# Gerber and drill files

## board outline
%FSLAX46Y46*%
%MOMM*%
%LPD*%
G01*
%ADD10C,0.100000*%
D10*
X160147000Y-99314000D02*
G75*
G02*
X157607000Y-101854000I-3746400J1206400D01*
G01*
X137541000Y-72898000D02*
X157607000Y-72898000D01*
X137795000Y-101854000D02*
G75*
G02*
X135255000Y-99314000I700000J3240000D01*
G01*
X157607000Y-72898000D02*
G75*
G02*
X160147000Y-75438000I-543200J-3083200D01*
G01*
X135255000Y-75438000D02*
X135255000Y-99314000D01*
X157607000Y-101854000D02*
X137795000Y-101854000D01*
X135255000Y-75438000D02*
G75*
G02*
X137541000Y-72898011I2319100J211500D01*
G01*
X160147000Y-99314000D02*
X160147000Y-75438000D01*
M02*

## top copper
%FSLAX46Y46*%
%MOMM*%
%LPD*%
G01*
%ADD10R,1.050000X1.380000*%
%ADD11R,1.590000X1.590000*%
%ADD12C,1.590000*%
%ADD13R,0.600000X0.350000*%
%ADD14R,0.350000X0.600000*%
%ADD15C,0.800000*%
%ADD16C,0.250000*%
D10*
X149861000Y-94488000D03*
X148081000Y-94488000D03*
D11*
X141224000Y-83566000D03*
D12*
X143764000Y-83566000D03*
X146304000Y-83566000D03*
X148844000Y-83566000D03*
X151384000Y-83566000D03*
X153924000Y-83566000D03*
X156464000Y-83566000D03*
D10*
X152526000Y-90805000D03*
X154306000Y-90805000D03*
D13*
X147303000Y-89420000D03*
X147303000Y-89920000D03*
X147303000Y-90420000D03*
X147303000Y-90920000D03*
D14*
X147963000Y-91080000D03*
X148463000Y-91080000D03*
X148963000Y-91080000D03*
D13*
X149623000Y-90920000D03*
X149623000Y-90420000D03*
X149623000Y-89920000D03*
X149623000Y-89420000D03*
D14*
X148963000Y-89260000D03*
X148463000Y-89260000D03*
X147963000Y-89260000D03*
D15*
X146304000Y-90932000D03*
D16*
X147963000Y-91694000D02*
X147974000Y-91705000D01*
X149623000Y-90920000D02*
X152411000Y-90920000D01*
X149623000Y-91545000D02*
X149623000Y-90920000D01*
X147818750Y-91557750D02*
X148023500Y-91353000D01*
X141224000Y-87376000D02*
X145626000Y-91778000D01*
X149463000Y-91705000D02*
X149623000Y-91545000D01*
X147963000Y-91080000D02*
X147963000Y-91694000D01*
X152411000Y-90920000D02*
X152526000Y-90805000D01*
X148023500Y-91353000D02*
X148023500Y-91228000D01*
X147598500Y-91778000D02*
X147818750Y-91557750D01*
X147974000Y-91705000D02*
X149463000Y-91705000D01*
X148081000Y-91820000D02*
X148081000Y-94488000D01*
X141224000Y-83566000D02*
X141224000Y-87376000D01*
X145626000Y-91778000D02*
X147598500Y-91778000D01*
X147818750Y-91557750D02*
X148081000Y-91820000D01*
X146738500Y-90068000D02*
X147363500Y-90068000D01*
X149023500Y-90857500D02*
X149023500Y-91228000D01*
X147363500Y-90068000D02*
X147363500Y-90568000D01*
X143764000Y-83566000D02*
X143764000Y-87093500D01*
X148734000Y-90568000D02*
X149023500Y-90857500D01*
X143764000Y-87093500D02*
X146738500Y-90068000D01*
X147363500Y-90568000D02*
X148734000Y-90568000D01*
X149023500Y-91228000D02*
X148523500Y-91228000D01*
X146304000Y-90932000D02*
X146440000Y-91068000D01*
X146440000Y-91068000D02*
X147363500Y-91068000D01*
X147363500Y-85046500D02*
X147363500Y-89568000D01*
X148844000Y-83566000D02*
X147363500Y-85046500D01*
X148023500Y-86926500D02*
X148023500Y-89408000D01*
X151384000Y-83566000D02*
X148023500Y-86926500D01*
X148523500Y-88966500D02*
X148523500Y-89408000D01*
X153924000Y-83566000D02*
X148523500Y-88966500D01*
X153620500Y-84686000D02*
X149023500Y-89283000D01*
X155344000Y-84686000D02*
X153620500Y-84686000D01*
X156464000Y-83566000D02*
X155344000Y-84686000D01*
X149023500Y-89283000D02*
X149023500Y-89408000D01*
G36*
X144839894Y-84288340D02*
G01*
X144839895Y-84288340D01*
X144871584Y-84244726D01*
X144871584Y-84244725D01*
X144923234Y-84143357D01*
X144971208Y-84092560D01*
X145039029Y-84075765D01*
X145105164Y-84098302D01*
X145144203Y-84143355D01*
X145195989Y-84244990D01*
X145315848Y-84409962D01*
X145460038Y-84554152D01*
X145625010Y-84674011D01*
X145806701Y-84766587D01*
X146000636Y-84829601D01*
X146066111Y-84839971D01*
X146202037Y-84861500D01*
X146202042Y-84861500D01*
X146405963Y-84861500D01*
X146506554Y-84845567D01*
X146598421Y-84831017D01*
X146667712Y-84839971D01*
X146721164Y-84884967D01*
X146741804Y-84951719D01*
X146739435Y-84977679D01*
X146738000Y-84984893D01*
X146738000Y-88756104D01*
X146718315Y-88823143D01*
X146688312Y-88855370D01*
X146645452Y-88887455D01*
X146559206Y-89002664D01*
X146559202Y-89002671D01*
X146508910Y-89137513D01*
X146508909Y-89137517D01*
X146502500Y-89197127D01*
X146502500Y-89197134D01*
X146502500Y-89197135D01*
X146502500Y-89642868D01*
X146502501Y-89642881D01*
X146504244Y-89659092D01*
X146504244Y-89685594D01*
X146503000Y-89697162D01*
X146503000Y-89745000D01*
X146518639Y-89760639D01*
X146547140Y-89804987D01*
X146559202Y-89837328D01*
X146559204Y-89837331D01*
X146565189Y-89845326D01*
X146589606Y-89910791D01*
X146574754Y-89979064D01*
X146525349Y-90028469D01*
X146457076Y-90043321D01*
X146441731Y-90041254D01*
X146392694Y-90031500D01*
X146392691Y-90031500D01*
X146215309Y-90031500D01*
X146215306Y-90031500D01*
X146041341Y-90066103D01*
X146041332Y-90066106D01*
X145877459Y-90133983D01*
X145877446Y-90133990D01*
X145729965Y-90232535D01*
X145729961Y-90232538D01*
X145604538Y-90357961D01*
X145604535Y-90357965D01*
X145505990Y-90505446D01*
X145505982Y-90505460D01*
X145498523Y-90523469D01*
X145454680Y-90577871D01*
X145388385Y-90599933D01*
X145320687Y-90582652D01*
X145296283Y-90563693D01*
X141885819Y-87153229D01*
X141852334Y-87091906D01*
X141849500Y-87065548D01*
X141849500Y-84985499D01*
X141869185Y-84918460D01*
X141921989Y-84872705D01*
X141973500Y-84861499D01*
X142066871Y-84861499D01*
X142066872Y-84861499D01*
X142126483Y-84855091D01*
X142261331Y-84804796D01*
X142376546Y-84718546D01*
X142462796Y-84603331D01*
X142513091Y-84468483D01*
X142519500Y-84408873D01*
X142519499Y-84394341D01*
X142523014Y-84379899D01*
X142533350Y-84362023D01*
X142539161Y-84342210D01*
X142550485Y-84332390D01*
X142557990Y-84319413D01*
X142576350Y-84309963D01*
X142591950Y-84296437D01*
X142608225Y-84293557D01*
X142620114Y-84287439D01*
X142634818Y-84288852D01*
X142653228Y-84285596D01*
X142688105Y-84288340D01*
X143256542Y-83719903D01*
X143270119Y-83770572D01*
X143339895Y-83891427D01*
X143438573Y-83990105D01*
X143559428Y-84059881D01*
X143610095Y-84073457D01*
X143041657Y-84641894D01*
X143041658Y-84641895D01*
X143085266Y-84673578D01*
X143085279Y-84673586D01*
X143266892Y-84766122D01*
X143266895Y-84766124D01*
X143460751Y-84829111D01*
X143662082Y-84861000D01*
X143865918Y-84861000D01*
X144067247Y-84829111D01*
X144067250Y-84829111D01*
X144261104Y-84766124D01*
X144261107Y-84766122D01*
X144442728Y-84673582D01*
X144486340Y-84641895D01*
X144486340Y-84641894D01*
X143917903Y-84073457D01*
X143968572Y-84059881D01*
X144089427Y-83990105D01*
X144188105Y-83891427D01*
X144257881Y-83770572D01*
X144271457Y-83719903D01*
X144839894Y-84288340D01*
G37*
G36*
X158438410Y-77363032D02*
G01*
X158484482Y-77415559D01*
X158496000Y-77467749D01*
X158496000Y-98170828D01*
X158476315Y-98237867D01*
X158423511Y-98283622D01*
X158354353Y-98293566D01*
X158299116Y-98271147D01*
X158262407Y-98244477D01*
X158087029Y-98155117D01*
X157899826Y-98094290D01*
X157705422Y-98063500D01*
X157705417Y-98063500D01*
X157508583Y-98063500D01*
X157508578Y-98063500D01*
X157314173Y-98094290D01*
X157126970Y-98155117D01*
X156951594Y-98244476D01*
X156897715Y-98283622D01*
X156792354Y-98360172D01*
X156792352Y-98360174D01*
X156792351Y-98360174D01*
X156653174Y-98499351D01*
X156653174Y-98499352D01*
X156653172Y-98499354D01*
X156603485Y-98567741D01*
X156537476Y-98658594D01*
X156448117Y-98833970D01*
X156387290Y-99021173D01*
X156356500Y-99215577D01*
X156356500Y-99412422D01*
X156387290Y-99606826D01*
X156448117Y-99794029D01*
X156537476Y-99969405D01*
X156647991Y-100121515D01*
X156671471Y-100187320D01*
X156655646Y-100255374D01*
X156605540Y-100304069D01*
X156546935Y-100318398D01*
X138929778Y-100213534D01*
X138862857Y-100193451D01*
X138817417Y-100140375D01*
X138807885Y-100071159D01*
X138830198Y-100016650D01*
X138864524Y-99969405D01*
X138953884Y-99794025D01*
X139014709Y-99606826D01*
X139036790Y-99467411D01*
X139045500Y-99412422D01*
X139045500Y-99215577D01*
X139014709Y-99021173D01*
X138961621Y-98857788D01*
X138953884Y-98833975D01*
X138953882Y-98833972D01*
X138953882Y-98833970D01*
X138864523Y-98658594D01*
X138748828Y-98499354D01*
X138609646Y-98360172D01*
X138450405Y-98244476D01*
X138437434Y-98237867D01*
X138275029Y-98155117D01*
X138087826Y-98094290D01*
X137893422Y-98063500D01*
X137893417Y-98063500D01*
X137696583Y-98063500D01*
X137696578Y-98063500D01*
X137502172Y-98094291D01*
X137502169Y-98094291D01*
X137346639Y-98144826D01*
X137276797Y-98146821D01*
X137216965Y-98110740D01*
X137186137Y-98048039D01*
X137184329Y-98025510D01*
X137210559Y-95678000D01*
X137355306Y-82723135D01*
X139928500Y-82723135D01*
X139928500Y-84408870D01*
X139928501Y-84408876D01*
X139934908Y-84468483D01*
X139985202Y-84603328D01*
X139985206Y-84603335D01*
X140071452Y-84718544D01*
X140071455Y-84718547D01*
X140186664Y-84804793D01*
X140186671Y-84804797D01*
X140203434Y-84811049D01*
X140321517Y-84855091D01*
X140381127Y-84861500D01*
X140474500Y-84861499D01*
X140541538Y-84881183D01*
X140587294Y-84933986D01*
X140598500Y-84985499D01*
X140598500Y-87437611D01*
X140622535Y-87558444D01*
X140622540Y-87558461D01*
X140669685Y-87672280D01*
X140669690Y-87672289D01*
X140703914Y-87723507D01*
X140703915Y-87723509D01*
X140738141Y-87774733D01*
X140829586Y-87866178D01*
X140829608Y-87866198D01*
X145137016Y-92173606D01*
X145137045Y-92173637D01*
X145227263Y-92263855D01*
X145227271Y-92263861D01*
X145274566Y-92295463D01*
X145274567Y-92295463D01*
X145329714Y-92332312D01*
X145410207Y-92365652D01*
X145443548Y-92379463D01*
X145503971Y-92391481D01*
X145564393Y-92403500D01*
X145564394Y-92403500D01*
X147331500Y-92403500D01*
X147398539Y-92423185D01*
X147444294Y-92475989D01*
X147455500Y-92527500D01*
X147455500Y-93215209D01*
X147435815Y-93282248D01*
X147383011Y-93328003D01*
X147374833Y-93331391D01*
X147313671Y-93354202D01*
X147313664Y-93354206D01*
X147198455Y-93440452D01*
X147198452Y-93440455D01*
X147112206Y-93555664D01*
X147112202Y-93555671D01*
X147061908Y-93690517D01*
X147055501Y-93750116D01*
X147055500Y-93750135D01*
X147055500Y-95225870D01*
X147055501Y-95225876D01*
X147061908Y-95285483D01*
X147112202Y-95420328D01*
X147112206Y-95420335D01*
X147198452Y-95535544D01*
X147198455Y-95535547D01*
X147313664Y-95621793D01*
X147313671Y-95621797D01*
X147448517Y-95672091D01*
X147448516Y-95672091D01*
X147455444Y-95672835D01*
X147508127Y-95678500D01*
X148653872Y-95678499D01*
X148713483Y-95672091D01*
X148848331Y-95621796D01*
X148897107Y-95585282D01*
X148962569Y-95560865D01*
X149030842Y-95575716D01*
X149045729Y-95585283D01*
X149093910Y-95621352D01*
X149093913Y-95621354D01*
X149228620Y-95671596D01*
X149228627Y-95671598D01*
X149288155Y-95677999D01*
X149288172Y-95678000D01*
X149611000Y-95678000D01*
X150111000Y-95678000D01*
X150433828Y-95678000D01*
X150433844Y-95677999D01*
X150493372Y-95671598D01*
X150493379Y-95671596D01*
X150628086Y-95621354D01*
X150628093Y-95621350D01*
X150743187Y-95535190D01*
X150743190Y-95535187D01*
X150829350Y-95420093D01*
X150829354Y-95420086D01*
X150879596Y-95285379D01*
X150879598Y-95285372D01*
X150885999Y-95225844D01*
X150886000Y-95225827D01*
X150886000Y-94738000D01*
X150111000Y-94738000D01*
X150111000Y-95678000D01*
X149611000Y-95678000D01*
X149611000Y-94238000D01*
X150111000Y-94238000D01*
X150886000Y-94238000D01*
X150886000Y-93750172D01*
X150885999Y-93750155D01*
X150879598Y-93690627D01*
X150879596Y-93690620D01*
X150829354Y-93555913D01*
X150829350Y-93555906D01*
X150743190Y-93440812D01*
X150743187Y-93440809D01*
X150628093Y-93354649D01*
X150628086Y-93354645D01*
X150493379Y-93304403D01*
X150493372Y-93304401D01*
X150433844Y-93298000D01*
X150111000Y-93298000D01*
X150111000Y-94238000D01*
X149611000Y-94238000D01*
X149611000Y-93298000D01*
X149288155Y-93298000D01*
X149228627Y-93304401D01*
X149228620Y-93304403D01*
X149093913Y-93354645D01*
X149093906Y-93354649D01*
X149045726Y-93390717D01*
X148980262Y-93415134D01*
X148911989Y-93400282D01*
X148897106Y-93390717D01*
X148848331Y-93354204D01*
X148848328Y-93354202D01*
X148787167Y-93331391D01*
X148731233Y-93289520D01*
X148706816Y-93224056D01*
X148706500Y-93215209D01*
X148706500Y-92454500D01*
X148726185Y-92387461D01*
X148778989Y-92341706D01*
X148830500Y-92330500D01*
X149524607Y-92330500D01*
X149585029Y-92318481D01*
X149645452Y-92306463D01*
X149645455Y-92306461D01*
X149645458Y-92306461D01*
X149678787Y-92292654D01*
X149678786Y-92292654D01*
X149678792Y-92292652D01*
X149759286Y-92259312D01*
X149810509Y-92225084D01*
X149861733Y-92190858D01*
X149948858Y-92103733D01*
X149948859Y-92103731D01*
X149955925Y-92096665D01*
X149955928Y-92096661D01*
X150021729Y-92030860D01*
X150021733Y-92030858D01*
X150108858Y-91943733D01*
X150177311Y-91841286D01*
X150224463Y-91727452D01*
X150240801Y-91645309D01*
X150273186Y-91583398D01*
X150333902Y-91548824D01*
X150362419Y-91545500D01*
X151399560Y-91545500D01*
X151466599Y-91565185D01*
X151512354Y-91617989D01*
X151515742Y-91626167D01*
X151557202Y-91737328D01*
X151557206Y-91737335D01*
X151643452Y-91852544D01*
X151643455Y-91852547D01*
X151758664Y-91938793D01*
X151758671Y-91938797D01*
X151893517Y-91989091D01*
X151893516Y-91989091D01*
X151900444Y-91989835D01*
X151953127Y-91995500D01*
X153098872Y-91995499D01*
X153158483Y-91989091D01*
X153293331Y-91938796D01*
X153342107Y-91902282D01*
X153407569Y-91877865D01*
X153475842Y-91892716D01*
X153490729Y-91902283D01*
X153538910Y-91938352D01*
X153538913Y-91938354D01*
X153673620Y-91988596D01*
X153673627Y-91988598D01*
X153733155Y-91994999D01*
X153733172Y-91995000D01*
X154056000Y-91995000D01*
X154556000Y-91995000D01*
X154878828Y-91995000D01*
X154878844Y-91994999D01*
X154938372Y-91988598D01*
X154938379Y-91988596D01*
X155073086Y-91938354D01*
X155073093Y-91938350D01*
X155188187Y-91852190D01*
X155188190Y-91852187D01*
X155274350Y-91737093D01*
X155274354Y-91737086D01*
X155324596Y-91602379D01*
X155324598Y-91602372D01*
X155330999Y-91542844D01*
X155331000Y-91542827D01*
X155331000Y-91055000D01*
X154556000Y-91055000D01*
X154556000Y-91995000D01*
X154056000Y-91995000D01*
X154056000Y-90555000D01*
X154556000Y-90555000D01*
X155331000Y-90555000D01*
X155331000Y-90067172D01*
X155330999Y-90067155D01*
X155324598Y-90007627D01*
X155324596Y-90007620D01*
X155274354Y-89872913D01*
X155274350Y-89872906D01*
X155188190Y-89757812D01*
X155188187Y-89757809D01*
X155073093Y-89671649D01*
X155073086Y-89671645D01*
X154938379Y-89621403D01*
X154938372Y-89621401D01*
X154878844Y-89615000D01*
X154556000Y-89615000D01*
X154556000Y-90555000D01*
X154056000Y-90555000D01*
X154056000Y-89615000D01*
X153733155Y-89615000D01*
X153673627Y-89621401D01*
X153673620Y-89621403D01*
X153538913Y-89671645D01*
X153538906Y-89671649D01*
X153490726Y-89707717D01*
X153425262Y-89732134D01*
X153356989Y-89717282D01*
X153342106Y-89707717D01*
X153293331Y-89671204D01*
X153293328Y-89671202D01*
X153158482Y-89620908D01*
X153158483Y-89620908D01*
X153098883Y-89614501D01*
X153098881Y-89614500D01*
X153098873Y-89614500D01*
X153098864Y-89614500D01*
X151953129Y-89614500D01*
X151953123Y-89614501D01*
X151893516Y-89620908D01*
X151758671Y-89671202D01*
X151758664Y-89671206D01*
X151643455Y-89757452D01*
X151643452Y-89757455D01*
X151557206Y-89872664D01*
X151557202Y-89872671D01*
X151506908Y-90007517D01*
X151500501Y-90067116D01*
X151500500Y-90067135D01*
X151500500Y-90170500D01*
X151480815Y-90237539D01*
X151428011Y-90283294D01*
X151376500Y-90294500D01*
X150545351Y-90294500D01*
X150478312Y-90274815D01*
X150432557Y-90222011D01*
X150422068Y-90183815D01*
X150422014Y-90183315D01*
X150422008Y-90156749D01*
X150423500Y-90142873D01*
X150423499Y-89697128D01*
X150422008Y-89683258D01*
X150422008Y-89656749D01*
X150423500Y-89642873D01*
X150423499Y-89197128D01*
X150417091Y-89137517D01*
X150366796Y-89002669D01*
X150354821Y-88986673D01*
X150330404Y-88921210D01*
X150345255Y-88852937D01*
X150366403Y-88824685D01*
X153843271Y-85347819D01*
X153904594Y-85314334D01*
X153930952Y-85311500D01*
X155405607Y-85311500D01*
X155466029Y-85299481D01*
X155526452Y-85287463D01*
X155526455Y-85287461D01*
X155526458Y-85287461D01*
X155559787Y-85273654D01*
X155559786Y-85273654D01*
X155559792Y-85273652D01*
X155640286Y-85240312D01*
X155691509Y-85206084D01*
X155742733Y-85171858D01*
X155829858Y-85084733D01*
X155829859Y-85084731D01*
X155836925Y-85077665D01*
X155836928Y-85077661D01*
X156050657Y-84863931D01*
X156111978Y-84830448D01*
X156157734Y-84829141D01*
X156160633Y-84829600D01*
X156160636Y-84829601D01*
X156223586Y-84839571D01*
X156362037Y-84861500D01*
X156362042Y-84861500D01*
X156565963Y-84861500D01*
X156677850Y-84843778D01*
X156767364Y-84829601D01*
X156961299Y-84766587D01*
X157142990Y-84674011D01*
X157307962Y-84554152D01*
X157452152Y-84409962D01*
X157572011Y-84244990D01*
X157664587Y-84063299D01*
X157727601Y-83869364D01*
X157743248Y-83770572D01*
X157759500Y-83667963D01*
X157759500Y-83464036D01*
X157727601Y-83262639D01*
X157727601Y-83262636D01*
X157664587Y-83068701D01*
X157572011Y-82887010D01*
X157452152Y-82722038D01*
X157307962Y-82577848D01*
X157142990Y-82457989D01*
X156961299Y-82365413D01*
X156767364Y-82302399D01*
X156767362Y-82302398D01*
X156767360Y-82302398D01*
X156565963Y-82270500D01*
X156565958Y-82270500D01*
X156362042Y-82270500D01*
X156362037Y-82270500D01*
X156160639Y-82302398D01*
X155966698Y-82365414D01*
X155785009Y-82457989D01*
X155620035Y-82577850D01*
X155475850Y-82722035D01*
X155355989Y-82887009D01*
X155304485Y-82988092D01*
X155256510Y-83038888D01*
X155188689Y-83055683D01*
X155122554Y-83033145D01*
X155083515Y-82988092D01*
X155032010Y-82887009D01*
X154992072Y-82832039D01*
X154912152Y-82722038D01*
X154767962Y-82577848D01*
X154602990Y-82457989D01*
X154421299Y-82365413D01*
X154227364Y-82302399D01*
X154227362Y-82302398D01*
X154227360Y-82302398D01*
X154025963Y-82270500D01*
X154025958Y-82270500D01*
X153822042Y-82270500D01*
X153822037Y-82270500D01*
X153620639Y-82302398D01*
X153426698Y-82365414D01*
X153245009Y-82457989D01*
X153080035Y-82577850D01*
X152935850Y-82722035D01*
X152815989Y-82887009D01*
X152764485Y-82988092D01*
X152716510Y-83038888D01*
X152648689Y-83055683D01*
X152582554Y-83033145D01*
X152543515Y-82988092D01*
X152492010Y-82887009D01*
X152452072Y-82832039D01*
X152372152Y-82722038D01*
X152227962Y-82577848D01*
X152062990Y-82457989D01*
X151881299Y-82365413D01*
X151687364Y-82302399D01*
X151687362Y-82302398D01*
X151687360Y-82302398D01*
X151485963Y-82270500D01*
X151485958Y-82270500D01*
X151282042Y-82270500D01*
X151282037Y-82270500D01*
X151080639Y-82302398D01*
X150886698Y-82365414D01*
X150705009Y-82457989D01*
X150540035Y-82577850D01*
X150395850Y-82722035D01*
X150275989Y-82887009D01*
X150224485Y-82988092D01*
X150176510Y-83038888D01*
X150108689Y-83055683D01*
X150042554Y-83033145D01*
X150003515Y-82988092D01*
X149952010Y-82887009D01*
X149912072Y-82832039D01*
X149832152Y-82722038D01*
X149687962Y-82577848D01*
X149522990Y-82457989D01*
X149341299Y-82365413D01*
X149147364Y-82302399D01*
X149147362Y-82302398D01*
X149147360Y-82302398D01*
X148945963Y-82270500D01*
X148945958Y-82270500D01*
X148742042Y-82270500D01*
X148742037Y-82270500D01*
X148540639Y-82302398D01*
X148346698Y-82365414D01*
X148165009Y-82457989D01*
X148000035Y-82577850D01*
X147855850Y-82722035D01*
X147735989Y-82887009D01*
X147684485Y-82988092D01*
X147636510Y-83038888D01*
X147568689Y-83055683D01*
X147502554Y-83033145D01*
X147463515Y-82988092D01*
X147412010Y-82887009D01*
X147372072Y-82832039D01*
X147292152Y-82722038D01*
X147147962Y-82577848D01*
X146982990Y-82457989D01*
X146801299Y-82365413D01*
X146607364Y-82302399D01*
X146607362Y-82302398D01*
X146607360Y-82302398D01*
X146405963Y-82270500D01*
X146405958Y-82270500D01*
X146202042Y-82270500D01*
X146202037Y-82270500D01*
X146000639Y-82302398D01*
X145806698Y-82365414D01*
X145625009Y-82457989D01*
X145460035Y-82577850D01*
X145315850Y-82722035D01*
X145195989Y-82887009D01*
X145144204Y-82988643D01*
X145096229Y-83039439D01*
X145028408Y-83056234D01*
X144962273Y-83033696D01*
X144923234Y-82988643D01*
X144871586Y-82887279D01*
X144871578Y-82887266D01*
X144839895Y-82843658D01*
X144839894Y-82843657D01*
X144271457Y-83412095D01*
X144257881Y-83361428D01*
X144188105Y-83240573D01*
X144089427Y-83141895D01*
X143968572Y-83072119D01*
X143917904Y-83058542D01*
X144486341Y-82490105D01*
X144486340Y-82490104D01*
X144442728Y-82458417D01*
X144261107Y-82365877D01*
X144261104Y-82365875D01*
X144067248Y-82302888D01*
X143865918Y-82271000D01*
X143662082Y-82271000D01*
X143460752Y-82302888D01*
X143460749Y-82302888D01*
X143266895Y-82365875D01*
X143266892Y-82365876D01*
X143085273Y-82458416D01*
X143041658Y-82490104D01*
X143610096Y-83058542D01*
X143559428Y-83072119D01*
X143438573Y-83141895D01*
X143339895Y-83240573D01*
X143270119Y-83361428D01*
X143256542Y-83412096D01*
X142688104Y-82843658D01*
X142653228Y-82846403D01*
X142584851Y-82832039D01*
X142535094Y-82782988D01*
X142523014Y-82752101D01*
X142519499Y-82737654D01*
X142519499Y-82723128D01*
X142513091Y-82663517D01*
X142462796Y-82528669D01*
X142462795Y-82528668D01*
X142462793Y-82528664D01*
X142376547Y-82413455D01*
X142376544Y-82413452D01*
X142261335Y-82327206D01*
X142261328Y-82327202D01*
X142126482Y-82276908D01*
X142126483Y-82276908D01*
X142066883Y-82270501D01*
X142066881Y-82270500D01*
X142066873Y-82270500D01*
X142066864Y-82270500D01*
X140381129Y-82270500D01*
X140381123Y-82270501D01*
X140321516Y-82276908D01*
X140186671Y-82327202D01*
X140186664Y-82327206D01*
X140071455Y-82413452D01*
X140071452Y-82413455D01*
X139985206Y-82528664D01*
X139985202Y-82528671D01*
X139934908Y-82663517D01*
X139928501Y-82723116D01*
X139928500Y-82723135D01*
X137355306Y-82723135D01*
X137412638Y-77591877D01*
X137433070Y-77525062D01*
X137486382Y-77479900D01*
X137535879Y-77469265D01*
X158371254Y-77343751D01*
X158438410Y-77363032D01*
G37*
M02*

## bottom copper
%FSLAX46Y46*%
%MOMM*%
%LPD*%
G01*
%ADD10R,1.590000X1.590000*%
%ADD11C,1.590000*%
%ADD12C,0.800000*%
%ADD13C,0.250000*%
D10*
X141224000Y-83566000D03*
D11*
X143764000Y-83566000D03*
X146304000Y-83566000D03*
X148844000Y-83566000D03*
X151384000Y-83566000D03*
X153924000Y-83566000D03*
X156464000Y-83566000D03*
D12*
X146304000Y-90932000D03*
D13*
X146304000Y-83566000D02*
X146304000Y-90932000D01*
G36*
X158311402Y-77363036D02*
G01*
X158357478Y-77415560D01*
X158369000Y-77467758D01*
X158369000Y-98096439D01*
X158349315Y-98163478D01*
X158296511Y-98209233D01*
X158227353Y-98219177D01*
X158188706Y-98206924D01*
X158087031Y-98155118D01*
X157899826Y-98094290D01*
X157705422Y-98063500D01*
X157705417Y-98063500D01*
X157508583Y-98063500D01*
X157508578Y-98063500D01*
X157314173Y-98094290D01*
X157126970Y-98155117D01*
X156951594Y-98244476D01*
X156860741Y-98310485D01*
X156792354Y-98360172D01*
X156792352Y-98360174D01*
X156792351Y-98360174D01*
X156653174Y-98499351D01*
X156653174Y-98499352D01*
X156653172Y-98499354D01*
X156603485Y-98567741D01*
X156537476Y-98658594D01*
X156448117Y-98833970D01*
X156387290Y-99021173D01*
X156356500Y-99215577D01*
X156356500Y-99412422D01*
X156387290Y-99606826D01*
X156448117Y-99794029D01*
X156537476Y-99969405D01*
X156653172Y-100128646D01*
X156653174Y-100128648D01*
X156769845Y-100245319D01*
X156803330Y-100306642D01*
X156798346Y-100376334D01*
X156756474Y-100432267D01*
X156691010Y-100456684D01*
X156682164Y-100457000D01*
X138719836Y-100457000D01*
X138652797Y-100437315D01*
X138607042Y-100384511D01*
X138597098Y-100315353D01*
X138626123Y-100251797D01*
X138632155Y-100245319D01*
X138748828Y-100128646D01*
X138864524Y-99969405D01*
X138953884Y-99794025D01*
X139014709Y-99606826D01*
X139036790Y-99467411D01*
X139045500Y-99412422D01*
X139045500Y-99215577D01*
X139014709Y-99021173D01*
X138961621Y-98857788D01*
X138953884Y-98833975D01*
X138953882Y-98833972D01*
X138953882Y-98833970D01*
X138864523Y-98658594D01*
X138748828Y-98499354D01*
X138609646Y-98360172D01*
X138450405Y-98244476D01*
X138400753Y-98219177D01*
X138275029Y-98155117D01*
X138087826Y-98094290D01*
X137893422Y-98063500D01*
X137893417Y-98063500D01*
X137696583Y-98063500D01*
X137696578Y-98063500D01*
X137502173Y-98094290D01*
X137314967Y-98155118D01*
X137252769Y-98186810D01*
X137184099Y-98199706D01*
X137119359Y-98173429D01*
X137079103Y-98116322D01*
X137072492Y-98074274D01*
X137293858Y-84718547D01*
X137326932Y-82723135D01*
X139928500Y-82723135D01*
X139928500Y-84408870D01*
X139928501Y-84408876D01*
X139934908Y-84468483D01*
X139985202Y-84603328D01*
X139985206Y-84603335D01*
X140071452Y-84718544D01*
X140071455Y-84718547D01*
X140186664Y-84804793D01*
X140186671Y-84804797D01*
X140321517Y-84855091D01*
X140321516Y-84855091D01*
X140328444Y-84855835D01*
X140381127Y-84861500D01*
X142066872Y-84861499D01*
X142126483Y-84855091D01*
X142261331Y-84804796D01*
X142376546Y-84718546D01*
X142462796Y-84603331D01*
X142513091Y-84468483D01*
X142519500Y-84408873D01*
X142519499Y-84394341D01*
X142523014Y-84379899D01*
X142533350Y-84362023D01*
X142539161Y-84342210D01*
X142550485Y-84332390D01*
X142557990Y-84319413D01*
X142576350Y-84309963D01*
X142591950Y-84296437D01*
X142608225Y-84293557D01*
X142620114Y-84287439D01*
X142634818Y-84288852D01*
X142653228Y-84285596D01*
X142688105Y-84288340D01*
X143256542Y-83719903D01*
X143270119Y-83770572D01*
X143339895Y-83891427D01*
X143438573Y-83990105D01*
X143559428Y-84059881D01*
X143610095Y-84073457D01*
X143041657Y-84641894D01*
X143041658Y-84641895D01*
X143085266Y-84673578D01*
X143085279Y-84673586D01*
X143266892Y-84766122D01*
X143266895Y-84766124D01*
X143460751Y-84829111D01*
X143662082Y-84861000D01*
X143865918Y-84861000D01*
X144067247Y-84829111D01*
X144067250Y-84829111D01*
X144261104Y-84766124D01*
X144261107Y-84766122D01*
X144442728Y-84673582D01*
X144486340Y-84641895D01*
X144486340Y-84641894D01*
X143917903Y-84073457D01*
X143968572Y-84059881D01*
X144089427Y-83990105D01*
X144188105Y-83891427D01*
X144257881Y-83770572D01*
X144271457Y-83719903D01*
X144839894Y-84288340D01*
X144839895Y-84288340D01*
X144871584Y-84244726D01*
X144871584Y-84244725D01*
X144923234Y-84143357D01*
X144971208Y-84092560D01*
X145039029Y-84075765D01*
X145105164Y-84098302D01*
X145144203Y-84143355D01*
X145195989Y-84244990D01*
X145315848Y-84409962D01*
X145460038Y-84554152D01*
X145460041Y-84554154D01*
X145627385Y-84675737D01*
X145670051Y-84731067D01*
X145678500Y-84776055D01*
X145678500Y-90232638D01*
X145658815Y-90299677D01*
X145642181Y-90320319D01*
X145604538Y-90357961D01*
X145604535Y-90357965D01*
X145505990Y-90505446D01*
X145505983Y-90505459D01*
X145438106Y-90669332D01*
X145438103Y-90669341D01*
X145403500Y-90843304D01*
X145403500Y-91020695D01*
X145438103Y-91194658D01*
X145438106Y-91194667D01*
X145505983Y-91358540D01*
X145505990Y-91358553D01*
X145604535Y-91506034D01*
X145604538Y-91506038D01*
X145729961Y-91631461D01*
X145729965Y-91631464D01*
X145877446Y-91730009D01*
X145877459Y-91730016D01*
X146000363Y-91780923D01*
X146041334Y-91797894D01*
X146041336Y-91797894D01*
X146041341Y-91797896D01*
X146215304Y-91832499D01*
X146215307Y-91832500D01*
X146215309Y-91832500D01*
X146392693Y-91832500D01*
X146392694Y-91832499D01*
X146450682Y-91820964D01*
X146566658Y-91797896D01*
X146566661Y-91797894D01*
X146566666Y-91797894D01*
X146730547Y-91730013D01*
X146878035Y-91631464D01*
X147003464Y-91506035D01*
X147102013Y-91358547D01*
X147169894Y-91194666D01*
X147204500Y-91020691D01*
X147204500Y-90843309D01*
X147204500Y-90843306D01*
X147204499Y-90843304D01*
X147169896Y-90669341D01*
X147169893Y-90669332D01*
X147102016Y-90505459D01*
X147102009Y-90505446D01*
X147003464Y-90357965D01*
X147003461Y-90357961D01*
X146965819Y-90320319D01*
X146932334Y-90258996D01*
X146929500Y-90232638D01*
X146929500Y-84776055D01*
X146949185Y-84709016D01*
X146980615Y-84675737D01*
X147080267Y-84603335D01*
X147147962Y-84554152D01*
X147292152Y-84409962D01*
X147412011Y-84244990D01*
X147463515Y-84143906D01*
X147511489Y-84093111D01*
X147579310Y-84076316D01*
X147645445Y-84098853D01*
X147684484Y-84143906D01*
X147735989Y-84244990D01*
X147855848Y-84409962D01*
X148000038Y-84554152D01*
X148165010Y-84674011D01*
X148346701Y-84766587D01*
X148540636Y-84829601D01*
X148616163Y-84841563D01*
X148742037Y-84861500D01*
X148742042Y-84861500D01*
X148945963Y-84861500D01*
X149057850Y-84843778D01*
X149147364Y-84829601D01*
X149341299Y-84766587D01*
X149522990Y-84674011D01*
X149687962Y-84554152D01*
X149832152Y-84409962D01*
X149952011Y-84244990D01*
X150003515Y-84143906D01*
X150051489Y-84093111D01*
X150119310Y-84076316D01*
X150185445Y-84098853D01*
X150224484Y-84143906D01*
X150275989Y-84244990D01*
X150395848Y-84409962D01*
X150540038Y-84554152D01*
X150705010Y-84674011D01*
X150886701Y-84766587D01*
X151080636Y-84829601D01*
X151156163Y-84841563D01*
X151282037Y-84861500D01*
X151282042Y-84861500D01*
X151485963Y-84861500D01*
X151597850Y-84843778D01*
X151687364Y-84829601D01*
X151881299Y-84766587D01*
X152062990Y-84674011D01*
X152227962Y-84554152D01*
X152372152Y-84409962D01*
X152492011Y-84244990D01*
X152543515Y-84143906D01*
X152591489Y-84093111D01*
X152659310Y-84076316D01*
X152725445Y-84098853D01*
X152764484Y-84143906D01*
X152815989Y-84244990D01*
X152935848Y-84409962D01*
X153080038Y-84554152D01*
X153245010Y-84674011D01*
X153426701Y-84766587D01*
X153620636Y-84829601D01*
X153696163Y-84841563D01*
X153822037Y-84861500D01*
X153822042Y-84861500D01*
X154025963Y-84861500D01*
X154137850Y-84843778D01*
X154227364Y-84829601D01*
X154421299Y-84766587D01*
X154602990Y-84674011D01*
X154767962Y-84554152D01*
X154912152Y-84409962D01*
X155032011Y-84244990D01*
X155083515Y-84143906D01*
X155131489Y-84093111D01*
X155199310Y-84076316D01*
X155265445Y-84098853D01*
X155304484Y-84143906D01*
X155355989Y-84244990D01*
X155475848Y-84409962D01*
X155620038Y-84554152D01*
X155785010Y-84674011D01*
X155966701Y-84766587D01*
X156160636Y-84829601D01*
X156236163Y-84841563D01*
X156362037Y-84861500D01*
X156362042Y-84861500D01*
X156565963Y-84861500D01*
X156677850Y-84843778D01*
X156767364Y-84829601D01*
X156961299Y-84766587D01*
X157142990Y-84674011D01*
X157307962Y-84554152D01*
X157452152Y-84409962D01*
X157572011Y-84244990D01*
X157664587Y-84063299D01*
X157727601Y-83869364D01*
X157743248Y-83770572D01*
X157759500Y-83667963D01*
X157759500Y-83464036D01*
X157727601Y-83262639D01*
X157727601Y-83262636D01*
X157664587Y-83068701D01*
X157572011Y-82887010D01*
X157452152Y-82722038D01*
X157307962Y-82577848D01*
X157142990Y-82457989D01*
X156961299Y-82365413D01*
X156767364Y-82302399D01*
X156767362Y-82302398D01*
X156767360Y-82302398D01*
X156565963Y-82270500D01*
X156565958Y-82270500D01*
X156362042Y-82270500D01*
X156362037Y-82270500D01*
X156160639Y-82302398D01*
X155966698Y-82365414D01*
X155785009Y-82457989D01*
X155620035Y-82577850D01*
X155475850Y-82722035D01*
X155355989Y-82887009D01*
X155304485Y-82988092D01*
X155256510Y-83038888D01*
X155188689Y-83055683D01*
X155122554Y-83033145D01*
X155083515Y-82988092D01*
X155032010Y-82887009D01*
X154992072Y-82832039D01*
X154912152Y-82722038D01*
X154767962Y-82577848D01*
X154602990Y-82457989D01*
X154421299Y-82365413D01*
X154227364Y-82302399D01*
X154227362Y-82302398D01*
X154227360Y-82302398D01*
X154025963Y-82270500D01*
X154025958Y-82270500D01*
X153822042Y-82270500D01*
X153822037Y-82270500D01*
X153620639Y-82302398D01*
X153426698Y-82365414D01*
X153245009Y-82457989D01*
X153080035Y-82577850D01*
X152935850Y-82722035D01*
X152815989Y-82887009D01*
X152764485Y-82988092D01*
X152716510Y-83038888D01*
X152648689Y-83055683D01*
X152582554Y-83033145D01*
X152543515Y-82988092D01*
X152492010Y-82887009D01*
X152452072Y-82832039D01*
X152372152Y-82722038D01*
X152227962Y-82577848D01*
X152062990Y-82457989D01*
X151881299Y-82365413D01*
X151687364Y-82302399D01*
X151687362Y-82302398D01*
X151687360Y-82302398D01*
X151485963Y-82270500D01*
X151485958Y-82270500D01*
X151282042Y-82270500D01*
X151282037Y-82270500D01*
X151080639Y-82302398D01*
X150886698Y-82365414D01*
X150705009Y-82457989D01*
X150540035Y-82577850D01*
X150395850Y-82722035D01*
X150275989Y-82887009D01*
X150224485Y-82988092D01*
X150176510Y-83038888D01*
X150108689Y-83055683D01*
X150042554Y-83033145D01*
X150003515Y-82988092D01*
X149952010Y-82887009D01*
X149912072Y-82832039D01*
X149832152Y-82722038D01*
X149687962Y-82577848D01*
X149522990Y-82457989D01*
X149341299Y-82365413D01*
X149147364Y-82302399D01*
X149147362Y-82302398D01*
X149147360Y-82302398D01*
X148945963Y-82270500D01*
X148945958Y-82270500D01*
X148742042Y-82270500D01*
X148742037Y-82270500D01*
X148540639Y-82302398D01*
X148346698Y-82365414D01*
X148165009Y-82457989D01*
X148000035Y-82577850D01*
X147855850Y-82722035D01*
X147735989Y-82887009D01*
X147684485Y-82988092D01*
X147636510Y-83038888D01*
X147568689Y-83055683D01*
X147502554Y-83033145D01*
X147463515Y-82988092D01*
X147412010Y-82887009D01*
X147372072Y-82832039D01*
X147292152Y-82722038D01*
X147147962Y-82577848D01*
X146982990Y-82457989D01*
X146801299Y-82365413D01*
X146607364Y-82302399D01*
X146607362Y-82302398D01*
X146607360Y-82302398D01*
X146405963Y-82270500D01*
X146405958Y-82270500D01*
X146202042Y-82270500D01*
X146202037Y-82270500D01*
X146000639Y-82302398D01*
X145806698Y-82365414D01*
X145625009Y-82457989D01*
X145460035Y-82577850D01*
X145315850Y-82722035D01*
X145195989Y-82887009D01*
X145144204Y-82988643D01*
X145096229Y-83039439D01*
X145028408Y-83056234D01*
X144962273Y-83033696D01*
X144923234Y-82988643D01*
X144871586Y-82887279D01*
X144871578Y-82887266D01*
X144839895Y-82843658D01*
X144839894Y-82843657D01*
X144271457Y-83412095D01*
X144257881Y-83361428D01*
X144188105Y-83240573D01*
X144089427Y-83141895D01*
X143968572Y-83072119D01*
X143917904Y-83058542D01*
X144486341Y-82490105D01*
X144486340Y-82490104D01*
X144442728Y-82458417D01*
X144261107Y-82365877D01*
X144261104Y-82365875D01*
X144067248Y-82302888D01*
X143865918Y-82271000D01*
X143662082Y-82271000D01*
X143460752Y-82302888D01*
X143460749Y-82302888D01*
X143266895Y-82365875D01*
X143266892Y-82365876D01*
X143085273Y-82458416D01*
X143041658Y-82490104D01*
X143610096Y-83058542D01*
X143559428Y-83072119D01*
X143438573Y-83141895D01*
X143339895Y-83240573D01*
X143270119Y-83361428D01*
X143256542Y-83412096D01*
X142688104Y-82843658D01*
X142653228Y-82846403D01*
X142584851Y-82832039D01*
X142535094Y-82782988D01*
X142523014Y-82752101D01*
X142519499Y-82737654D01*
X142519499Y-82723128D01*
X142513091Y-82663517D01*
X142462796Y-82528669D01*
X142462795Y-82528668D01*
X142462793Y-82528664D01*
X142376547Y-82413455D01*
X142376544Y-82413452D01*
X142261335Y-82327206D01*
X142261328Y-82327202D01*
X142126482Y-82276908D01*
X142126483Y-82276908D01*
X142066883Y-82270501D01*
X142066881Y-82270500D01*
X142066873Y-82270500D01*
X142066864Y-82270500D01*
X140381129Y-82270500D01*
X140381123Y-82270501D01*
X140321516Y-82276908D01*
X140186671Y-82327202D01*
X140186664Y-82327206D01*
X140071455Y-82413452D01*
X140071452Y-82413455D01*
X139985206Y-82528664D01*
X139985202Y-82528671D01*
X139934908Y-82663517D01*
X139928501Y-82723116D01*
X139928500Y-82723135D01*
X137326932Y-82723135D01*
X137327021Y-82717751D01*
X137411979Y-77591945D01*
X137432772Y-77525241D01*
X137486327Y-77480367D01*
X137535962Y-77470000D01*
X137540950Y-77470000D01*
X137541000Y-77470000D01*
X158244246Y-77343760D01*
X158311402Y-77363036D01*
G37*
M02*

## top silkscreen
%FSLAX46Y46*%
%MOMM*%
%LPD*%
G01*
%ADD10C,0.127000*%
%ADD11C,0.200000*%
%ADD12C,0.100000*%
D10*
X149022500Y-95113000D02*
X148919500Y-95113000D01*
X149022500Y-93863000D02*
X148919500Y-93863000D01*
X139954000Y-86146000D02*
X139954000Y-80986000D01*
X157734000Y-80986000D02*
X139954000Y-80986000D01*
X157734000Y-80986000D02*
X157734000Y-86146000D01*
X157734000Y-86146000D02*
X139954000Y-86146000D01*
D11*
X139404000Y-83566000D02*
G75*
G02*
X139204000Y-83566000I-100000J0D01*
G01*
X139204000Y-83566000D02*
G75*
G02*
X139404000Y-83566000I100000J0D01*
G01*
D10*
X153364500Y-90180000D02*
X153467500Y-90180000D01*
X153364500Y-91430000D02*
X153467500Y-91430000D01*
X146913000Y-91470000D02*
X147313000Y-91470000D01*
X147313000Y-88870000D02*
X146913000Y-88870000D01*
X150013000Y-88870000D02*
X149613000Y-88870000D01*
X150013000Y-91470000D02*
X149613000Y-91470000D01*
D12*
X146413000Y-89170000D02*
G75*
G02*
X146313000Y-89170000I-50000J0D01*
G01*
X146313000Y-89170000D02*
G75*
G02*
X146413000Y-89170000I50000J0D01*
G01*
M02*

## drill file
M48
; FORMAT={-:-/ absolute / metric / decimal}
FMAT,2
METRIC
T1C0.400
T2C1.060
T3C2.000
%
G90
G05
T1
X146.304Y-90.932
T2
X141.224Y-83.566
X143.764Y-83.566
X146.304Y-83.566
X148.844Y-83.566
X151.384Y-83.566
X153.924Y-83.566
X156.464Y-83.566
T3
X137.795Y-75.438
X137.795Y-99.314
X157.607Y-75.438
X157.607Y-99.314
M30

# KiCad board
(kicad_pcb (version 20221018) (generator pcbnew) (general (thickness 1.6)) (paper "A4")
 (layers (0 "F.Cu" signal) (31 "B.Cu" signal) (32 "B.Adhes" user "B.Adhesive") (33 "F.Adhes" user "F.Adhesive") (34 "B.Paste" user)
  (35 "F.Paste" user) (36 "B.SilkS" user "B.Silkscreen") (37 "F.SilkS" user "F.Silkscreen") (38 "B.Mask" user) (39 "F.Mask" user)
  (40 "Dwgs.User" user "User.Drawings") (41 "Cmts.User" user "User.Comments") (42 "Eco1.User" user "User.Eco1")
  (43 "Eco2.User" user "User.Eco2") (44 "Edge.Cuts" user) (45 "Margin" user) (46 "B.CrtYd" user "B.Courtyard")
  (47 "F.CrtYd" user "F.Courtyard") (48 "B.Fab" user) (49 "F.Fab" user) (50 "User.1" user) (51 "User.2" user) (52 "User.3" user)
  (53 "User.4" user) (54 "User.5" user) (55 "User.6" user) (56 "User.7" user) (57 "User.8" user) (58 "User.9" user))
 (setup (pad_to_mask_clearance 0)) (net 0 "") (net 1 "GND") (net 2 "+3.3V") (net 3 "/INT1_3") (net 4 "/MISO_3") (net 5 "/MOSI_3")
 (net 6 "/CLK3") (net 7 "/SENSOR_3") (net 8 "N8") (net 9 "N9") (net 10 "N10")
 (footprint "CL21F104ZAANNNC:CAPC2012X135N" (layer "F.Cu") (at 148.971 94.488 180)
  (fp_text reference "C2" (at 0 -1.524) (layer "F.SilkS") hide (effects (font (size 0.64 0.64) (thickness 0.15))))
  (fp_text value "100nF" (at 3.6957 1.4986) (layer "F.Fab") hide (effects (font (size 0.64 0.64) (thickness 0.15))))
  (fp_line (start -0.0515 -0.625) (end 0.0515 -0.625) (stroke (width 0.127) (type solid)) (layer "F.SilkS"))
  (fp_line (start -0.0515 0.625) (end 0.0515 0.625) (stroke (width 0.127) (type solid)) (layer "F.SilkS"))
  (pad "1" smd rect (at -0.89 0 180) (size 1.05 1.38) (layers "F.Cu" "F.Paste" "F.Mask") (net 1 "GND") (solder_mask_margin 0.102))
  (pad "2" smd rect (at 0.89 0 180) (size 1.05 1.38) (layers "F.Cu" "F.Paste" "F.Mask") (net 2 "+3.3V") (solder_mask_margin 0.102)))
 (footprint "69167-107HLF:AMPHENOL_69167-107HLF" (layer "F.Cu") (at 148.844 83.566)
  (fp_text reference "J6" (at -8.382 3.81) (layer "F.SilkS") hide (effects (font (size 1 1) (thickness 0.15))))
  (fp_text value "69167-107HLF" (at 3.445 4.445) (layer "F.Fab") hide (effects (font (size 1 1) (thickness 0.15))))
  (fp_line (start -8.89 2.58) (end -8.89 -2.58) (stroke (width 0.127) (type solid)) (layer "F.SilkS"))
  (fp_line (start 8.89 -2.58) (end -8.89 -2.58) (stroke (width 0.127) (type solid)) (layer "F.SilkS"))
  (fp_line (start 8.89 -2.58) (end 8.89 2.58) (stroke (width 0.127) (type solid)) (layer "F.SilkS"))
  (fp_line (start 8.89 2.58) (end -8.89 2.58) (stroke (width 0.127) (type solid)) (layer "F.SilkS"))
  (fp_circle (center -9.54 0) (end -9.44 0) (stroke (width 0.2) (type solid)) (fill none) (layer "F.SilkS"))
  (pad "01" thru_hole rect (at -7.62 0) (size 1.59 1.59) (drill 1.06) (layers "*.Cu" "*.Mask") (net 2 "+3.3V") (solder_mask_margin 0.102))
  (pad "02" thru_hole circle (at -5.08 0) (size 1.59 1.59) (drill 1.06) (layers "*.Cu" "*.Mask") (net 1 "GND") (solder_mask_margin 0.102))
  (pad "03" thru_hole circle (at -2.54 0) (size 1.59 1.59) (drill 1.06) (layers "*.Cu" "*.Mask") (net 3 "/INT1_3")
   (solder_mask_margin 0.102))
  (pad "04" thru_hole circle (at 0 0) (size 1.59 1.59) (drill 1.06) (layers "*.Cu" "*.Mask") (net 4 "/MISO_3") (solder_mask_margin 0.102))
  (pad "05" thru_hole circle (at 2.54 0) (size 1.59 1.59) (drill 1.06) (layers "*.Cu" "*.Mask") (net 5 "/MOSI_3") (solder_mask_margin 0.102))
  (pad "06" thru_hole circle (at 5.08 0) (size 1.59 1.59) (drill 1.06) (layers "*.Cu" "*.Mask") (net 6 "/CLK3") (solder_mask_margin 0.102))
  (pad "07" thru_hole circle (at 7.62 0) (size 1.59 1.59) (drill 1.06) (layers "*.Cu" "*.Mask") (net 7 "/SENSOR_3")
   (solder_mask_margin 0.102)))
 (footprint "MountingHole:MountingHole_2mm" (layer "F.Cu") (at 137.795 75.438)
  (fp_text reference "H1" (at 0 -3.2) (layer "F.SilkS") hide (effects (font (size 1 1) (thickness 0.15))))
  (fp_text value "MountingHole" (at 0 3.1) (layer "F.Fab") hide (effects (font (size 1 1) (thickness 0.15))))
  (pad "" np_thru_hole circle (at 0 0) (size 2 2) (drill 2) (layers "*.Cu" "*.Mask")))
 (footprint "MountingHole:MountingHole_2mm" (layer "F.Cu") (at 157.607 75.438)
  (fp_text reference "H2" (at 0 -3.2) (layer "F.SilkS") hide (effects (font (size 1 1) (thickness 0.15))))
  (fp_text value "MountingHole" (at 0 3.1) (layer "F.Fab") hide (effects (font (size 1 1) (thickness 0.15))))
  (pad "" np_thru_hole circle (at 0 0) (size 2 2) (drill 2) (layers "*.Cu" "*.Mask")))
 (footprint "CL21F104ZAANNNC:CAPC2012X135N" (layer "F.Cu") (at 153.416 90.805)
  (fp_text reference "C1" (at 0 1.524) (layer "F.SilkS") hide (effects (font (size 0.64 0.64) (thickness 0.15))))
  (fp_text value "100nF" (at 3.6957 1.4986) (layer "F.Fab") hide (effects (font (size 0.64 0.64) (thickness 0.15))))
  (fp_line (start -0.0515 -0.625) (end 0.0515 -0.625) (stroke (width 0.127) (type solid)) (layer "F.SilkS"))
  (fp_line (start -0.0515 0.625) (end 0.0515 0.625) (stroke (width 0.127) (type solid)) (layer "F.SilkS"))
  (pad "1" smd rect (at -0.89 0) (size 1.05 1.38) (layers "F.Cu" "F.Paste" "F.Mask") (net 2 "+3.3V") (solder_mask_margin 0.102))
  (pad "2" smd rect (at 0.89 0) (size 1.05 1.38) (layers "F.Cu" "F.Paste" "F.Mask") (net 1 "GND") (solder_mask_margin 0.102)))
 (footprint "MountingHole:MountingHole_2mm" (layer "F.Cu") (at 157.607 99.314)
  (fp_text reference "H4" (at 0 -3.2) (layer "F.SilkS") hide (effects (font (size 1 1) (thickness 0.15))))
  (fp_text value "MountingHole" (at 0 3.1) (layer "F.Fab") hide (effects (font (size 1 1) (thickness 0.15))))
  (pad "" np_thru_hole circle (at 0 0) (size 2 2) (drill 2) (layers "*.Cu" "*.Mask")))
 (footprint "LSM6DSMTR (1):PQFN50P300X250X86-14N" (layer "F.Cu") (at 148.463 90.17)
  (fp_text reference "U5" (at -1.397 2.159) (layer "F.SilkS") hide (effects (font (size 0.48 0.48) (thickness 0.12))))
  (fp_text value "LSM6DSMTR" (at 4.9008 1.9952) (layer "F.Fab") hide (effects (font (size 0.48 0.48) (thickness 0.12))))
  (fp_line (start -1.55 1.3) (end -1.15 1.3) (stroke (width 0.127) (type solid)) (layer "F.SilkS"))
  (fp_line (start -1.15 -1.3) (end -1.55 -1.3) (stroke (width 0.127) (type solid)) (layer "F.SilkS"))
  (fp_line (start 1.55 -1.3) (end 1.15 -1.3) (stroke (width 0.127) (type solid)) (layer "F.SilkS"))
  (fp_line (start 1.55 1.3) (end 1.15 1.3) (stroke (width 0.127) (type solid)) (layer "F.SilkS"))
  (fp_circle (center -2.1 -1) (end -2.05 -1) (stroke (width 0.1) (type solid)) (fill none) (layer "F.SilkS"))
  (pad "1" smd rect (at -1.16 -0.75) (size 0.6 0.35) (layers "F.Cu" "F.Paste" "F.Mask") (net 4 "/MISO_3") (solder_mask_margin 0.102))
  (pad "2" smd rect (at -1.16 -0.25) (size 0.6 0.35) (layers "F.Cu" "F.Paste" "F.Mask") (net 1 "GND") (solder_mask_margin 0.102))
  (pad "3" smd rect (at -1.16 0.25) (size 0.6 0.35) (layers "F.Cu" "F.Paste" "F.Mask") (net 1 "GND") (solder_mask_margin 0.102))
  (pad "4" smd rect (at -1.16 0.75) (size 0.6 0.35) (layers "F.Cu" "F.Paste" "F.Mask") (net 3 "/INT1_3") (solder_mask_margin 0.102))
  (pad "5" smd rect (at -0.5 0.91 90) (size 0.6 0.35) (layers "F.Cu" "F.Paste" "F.Mask") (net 2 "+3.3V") (solder_mask_margin 0.102))
  (pad "6" smd rect (at 0 0.91 90) (size 0.6 0.35) (layers "F.Cu" "F.Paste" "F.Mask") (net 1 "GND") (solder_mask_margin 0.102))
  (pad "7" smd rect (at 0.5 0.91 90) (size 0.6 0.35) (layers "F.Cu" "F.Paste" "F.Mask") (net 1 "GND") (solder_mask_margin 0.102))
  (pad "8" smd rect (at 1.16 0.75) (size 0.6 0.35) (layers "F.Cu" "F.Paste" "F.Mask") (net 2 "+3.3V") (solder_mask_margin 0.102))
  (pad "9" smd rect (at 1.16 0.25) (size 0.6 0.35) (layers "F.Cu" "F.Paste" "F.Mask") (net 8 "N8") (solder_mask_margin 0.102))
  (pad "10" smd rect (at 1.16 -0.25) (size 0.6 0.35) (layers "F.Cu" "F.Paste" "F.Mask") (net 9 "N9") (solder_mask_margin 0.102))
  (pad "11" smd rect (at 1.16 -0.75) (size 0.6 0.35) (layers "F.Cu" "F.Paste" "F.Mask") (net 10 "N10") (solder_mask_margin 0.102))
  (pad "12" smd rect (at 0.5 -0.91 90) (size 0.6 0.35) (layers "F.Cu" "F.Paste" "F.Mask") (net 7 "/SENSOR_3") (solder_mask_margin 0.102))
  (pad "13" smd rect (at 0 -0.91 90) (size 0.6 0.35) (layers "F.Cu" "F.Paste" "F.Mask") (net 6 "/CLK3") (solder_mask_margin 0.102))
  (pad "14" smd rect (at -0.5 -0.91 90) (size 0.6 0.35) (layers "F.Cu" "F.Paste" "F.Mask") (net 5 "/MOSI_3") (solder_mask_margin 0.102)))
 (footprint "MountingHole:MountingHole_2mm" (layer "F.Cu") (at 137.795 99.314)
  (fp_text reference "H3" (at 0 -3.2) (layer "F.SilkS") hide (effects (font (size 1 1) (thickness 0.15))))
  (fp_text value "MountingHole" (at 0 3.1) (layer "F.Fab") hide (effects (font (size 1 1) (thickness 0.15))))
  (pad "" np_thru_hole circle (at 0 0) (size 2 2) (drill 2) (layers "*.Cu" "*.Mask")))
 (gr_arc (start 160.147 99.314) (mid 159.183666 100.890666) (end 157.607 101.854) (stroke (width 0.1) (type default)) (layer "Edge.Cuts"))
 (gr_line (start 137.541 72.898) (end 157.607 72.898) (stroke (width 0.1) (type default)) (layer "Edge.Cuts"))
 (gr_arc (start 137.795 101.854) (mid 136.151114 100.957886) (end 135.255 99.314) (stroke (width 0.1) (type default)) (layer "Edge.Cuts"))
 (gr_arc (start 157.607 72.898) (mid 159.277529 73.767471) (end 160.147 75.438) (stroke (width 0.1) (type default)) (layer "Edge.Cuts"))
 (gr_line (start 135.255 75.438) (end 135.255 99.314) (stroke (width 0.1) (type default)) (layer "Edge.Cuts"))
 (gr_line (start 157.607 101.854) (end 137.795 101.854) (stroke (width 0.1) (type default)) (layer "Edge.Cuts"))
 (gr_arc (start 135.255 75.438) (mid 135.843178 73.66866) (end 137.541 72.898) (stroke (width 0.1) (type default)) (layer "Edge.Cuts"))
 (gr_line (start 160.147 99.314) (end 160.147 75.438) (stroke (width 0.1) (type default)) (layer "Edge.Cuts"))
 (segment (start 147.963 91.694) (end 147.974 91.705) (width 0.25) (layer "F.Cu") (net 2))
 (segment (start 149.623 90.92) (end 152.411 90.92) (width 0.25) (layer "F.Cu") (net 2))
 (segment (start 149.623 91.545) (end 149.623 90.92) (width 0.25) (layer "F.Cu") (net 2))
 (segment (start 147.81875 91.55775) (end 148.0235 91.353) (width 0.25) (layer "F.Cu") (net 2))
 (segment (start 141.224 87.376) (end 145.626 91.778) (width 0.25) (layer "F.Cu") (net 2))
 (segment (start 149.463 91.705) (end 149.623 91.545) (width 0.25) (layer "F.Cu") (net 2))
 (segment (start 147.963 91.08) (end 147.963 91.694) (width 0.25) (layer "F.Cu") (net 2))
 (segment (start 152.411 90.92) (end 152.526 90.805) (width 0.25) (layer "F.Cu") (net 2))
 (segment (start 148.0235 91.353) (end 148.0235 91.228) (width 0.25) (layer "F.Cu") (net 2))
 (segment (start 147.5985 91.778) (end 147.81875 91.55775) (width 0.25) (layer "F.Cu") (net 2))
 (segment (start 147.974 91.705) (end 149.463 91.705) (width 0.25) (layer "F.Cu") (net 2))
 (segment (start 148.081 91.82) (end 148.081 94.488) (width 0.25) (layer "F.Cu") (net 2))
 (segment (start 141.224 83.566) (end 141.224 87.376) (width 0.25) (layer "F.Cu") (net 2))
 (segment (start 145.626 91.778) (end 147.5985 91.778) (width 0.25) (layer "F.Cu") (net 2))
 (segment (start 147.81875 91.55775) (end 148.081 91.82) (width 0.25) (layer "F.Cu") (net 2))
 (segment (start 146.7385 90.068) (end 147.3635 90.068) (width 0.25) (layer "F.Cu") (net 1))
 (segment (start 149.0235 90.8575) (end 149.0235 91.228) (width 0.25) (layer "F.Cu") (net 1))
 (segment (start 147.3635 90.068) (end 147.3635 90.568) (width 0.25) (layer "F.Cu") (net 1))
 (segment (start 143.764 83.566) (end 143.764 87.0935) (width 0.25) (layer "F.Cu") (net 1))
 (segment (start 148.734 90.568) (end 149.0235 90.8575) (width 0.25) (layer "F.Cu") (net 1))
 (segment (start 143.764 87.0935) (end 146.7385 90.068) (width 0.25) (layer "F.Cu") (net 1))
 (segment (start 147.3635 90.568) (end 148.734 90.568) (width 0.25) (layer "F.Cu") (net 1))
 (segment (start 149.0235 91.228) (end 148.5235 91.228) (width 0.25) (layer "F.Cu") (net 1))
 (segment (start 146.304 90.932) (end 146.44 91.068) (width 0.25) (layer "F.Cu") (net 3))
 (segment (start 146.44 91.068) (end 147.3635 91.068) (width 0.25) (layer "F.Cu") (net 3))
 (via (at 146.304 90.932) (size 0.8) (drill 0.4) (layers "F.Cu" "B.Cu") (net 3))
 (segment (start 146.304 83.566) (end 146.304 90.932) (width 0.25) (layer "B.Cu") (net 3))
 (segment (start 147.3635 85.0465) (end 147.3635 89.568) (width 0.25) (layer "F.Cu") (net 4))
 (segment (start 148.844 83.566) (end 147.3635 85.0465) (width 0.25) (layer "F.Cu") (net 4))
 (segment (start 148.0235 86.9265) (end 148.0235 89.408) (width 0.25) (layer "F.Cu") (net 5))
 (segment (start 151.384 83.566) (end 148.0235 86.9265) (width 0.25) (layer "F.Cu") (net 5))
 (segment (start 148.5235 88.9665) (end 148.5235 89.408) (width 0.25) (layer "F.Cu") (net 6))
 (segment (start 153.924 83.566) (end 148.5235 88.9665) (width 0.25) (layer "F.Cu") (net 6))
 (segment (start 153.6205 84.686) (end 149.0235 89.283) (width 0.25) (layer "F.Cu") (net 7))
 (segment (start 155.344 84.686) (end 153.6205 84.686) (width 0.25) (layer "F.Cu") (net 7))
 (segment (start 156.464 83.566) (end 155.344 84.686) (width 0.25) (layer "F.Cu") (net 7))
 (segment (start 149.0235 89.283) (end 149.0235 89.408) (width 0.25) (layer "F.Cu") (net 7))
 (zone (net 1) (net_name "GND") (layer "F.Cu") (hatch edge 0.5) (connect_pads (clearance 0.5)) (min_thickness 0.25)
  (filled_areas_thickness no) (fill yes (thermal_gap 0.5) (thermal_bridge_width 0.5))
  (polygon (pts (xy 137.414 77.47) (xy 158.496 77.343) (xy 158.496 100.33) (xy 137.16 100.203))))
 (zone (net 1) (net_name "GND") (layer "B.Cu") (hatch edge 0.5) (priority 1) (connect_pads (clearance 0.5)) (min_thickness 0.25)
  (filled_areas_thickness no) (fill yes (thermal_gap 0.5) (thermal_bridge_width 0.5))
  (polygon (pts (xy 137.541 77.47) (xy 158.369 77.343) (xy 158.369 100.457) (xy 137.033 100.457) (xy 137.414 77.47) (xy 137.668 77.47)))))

